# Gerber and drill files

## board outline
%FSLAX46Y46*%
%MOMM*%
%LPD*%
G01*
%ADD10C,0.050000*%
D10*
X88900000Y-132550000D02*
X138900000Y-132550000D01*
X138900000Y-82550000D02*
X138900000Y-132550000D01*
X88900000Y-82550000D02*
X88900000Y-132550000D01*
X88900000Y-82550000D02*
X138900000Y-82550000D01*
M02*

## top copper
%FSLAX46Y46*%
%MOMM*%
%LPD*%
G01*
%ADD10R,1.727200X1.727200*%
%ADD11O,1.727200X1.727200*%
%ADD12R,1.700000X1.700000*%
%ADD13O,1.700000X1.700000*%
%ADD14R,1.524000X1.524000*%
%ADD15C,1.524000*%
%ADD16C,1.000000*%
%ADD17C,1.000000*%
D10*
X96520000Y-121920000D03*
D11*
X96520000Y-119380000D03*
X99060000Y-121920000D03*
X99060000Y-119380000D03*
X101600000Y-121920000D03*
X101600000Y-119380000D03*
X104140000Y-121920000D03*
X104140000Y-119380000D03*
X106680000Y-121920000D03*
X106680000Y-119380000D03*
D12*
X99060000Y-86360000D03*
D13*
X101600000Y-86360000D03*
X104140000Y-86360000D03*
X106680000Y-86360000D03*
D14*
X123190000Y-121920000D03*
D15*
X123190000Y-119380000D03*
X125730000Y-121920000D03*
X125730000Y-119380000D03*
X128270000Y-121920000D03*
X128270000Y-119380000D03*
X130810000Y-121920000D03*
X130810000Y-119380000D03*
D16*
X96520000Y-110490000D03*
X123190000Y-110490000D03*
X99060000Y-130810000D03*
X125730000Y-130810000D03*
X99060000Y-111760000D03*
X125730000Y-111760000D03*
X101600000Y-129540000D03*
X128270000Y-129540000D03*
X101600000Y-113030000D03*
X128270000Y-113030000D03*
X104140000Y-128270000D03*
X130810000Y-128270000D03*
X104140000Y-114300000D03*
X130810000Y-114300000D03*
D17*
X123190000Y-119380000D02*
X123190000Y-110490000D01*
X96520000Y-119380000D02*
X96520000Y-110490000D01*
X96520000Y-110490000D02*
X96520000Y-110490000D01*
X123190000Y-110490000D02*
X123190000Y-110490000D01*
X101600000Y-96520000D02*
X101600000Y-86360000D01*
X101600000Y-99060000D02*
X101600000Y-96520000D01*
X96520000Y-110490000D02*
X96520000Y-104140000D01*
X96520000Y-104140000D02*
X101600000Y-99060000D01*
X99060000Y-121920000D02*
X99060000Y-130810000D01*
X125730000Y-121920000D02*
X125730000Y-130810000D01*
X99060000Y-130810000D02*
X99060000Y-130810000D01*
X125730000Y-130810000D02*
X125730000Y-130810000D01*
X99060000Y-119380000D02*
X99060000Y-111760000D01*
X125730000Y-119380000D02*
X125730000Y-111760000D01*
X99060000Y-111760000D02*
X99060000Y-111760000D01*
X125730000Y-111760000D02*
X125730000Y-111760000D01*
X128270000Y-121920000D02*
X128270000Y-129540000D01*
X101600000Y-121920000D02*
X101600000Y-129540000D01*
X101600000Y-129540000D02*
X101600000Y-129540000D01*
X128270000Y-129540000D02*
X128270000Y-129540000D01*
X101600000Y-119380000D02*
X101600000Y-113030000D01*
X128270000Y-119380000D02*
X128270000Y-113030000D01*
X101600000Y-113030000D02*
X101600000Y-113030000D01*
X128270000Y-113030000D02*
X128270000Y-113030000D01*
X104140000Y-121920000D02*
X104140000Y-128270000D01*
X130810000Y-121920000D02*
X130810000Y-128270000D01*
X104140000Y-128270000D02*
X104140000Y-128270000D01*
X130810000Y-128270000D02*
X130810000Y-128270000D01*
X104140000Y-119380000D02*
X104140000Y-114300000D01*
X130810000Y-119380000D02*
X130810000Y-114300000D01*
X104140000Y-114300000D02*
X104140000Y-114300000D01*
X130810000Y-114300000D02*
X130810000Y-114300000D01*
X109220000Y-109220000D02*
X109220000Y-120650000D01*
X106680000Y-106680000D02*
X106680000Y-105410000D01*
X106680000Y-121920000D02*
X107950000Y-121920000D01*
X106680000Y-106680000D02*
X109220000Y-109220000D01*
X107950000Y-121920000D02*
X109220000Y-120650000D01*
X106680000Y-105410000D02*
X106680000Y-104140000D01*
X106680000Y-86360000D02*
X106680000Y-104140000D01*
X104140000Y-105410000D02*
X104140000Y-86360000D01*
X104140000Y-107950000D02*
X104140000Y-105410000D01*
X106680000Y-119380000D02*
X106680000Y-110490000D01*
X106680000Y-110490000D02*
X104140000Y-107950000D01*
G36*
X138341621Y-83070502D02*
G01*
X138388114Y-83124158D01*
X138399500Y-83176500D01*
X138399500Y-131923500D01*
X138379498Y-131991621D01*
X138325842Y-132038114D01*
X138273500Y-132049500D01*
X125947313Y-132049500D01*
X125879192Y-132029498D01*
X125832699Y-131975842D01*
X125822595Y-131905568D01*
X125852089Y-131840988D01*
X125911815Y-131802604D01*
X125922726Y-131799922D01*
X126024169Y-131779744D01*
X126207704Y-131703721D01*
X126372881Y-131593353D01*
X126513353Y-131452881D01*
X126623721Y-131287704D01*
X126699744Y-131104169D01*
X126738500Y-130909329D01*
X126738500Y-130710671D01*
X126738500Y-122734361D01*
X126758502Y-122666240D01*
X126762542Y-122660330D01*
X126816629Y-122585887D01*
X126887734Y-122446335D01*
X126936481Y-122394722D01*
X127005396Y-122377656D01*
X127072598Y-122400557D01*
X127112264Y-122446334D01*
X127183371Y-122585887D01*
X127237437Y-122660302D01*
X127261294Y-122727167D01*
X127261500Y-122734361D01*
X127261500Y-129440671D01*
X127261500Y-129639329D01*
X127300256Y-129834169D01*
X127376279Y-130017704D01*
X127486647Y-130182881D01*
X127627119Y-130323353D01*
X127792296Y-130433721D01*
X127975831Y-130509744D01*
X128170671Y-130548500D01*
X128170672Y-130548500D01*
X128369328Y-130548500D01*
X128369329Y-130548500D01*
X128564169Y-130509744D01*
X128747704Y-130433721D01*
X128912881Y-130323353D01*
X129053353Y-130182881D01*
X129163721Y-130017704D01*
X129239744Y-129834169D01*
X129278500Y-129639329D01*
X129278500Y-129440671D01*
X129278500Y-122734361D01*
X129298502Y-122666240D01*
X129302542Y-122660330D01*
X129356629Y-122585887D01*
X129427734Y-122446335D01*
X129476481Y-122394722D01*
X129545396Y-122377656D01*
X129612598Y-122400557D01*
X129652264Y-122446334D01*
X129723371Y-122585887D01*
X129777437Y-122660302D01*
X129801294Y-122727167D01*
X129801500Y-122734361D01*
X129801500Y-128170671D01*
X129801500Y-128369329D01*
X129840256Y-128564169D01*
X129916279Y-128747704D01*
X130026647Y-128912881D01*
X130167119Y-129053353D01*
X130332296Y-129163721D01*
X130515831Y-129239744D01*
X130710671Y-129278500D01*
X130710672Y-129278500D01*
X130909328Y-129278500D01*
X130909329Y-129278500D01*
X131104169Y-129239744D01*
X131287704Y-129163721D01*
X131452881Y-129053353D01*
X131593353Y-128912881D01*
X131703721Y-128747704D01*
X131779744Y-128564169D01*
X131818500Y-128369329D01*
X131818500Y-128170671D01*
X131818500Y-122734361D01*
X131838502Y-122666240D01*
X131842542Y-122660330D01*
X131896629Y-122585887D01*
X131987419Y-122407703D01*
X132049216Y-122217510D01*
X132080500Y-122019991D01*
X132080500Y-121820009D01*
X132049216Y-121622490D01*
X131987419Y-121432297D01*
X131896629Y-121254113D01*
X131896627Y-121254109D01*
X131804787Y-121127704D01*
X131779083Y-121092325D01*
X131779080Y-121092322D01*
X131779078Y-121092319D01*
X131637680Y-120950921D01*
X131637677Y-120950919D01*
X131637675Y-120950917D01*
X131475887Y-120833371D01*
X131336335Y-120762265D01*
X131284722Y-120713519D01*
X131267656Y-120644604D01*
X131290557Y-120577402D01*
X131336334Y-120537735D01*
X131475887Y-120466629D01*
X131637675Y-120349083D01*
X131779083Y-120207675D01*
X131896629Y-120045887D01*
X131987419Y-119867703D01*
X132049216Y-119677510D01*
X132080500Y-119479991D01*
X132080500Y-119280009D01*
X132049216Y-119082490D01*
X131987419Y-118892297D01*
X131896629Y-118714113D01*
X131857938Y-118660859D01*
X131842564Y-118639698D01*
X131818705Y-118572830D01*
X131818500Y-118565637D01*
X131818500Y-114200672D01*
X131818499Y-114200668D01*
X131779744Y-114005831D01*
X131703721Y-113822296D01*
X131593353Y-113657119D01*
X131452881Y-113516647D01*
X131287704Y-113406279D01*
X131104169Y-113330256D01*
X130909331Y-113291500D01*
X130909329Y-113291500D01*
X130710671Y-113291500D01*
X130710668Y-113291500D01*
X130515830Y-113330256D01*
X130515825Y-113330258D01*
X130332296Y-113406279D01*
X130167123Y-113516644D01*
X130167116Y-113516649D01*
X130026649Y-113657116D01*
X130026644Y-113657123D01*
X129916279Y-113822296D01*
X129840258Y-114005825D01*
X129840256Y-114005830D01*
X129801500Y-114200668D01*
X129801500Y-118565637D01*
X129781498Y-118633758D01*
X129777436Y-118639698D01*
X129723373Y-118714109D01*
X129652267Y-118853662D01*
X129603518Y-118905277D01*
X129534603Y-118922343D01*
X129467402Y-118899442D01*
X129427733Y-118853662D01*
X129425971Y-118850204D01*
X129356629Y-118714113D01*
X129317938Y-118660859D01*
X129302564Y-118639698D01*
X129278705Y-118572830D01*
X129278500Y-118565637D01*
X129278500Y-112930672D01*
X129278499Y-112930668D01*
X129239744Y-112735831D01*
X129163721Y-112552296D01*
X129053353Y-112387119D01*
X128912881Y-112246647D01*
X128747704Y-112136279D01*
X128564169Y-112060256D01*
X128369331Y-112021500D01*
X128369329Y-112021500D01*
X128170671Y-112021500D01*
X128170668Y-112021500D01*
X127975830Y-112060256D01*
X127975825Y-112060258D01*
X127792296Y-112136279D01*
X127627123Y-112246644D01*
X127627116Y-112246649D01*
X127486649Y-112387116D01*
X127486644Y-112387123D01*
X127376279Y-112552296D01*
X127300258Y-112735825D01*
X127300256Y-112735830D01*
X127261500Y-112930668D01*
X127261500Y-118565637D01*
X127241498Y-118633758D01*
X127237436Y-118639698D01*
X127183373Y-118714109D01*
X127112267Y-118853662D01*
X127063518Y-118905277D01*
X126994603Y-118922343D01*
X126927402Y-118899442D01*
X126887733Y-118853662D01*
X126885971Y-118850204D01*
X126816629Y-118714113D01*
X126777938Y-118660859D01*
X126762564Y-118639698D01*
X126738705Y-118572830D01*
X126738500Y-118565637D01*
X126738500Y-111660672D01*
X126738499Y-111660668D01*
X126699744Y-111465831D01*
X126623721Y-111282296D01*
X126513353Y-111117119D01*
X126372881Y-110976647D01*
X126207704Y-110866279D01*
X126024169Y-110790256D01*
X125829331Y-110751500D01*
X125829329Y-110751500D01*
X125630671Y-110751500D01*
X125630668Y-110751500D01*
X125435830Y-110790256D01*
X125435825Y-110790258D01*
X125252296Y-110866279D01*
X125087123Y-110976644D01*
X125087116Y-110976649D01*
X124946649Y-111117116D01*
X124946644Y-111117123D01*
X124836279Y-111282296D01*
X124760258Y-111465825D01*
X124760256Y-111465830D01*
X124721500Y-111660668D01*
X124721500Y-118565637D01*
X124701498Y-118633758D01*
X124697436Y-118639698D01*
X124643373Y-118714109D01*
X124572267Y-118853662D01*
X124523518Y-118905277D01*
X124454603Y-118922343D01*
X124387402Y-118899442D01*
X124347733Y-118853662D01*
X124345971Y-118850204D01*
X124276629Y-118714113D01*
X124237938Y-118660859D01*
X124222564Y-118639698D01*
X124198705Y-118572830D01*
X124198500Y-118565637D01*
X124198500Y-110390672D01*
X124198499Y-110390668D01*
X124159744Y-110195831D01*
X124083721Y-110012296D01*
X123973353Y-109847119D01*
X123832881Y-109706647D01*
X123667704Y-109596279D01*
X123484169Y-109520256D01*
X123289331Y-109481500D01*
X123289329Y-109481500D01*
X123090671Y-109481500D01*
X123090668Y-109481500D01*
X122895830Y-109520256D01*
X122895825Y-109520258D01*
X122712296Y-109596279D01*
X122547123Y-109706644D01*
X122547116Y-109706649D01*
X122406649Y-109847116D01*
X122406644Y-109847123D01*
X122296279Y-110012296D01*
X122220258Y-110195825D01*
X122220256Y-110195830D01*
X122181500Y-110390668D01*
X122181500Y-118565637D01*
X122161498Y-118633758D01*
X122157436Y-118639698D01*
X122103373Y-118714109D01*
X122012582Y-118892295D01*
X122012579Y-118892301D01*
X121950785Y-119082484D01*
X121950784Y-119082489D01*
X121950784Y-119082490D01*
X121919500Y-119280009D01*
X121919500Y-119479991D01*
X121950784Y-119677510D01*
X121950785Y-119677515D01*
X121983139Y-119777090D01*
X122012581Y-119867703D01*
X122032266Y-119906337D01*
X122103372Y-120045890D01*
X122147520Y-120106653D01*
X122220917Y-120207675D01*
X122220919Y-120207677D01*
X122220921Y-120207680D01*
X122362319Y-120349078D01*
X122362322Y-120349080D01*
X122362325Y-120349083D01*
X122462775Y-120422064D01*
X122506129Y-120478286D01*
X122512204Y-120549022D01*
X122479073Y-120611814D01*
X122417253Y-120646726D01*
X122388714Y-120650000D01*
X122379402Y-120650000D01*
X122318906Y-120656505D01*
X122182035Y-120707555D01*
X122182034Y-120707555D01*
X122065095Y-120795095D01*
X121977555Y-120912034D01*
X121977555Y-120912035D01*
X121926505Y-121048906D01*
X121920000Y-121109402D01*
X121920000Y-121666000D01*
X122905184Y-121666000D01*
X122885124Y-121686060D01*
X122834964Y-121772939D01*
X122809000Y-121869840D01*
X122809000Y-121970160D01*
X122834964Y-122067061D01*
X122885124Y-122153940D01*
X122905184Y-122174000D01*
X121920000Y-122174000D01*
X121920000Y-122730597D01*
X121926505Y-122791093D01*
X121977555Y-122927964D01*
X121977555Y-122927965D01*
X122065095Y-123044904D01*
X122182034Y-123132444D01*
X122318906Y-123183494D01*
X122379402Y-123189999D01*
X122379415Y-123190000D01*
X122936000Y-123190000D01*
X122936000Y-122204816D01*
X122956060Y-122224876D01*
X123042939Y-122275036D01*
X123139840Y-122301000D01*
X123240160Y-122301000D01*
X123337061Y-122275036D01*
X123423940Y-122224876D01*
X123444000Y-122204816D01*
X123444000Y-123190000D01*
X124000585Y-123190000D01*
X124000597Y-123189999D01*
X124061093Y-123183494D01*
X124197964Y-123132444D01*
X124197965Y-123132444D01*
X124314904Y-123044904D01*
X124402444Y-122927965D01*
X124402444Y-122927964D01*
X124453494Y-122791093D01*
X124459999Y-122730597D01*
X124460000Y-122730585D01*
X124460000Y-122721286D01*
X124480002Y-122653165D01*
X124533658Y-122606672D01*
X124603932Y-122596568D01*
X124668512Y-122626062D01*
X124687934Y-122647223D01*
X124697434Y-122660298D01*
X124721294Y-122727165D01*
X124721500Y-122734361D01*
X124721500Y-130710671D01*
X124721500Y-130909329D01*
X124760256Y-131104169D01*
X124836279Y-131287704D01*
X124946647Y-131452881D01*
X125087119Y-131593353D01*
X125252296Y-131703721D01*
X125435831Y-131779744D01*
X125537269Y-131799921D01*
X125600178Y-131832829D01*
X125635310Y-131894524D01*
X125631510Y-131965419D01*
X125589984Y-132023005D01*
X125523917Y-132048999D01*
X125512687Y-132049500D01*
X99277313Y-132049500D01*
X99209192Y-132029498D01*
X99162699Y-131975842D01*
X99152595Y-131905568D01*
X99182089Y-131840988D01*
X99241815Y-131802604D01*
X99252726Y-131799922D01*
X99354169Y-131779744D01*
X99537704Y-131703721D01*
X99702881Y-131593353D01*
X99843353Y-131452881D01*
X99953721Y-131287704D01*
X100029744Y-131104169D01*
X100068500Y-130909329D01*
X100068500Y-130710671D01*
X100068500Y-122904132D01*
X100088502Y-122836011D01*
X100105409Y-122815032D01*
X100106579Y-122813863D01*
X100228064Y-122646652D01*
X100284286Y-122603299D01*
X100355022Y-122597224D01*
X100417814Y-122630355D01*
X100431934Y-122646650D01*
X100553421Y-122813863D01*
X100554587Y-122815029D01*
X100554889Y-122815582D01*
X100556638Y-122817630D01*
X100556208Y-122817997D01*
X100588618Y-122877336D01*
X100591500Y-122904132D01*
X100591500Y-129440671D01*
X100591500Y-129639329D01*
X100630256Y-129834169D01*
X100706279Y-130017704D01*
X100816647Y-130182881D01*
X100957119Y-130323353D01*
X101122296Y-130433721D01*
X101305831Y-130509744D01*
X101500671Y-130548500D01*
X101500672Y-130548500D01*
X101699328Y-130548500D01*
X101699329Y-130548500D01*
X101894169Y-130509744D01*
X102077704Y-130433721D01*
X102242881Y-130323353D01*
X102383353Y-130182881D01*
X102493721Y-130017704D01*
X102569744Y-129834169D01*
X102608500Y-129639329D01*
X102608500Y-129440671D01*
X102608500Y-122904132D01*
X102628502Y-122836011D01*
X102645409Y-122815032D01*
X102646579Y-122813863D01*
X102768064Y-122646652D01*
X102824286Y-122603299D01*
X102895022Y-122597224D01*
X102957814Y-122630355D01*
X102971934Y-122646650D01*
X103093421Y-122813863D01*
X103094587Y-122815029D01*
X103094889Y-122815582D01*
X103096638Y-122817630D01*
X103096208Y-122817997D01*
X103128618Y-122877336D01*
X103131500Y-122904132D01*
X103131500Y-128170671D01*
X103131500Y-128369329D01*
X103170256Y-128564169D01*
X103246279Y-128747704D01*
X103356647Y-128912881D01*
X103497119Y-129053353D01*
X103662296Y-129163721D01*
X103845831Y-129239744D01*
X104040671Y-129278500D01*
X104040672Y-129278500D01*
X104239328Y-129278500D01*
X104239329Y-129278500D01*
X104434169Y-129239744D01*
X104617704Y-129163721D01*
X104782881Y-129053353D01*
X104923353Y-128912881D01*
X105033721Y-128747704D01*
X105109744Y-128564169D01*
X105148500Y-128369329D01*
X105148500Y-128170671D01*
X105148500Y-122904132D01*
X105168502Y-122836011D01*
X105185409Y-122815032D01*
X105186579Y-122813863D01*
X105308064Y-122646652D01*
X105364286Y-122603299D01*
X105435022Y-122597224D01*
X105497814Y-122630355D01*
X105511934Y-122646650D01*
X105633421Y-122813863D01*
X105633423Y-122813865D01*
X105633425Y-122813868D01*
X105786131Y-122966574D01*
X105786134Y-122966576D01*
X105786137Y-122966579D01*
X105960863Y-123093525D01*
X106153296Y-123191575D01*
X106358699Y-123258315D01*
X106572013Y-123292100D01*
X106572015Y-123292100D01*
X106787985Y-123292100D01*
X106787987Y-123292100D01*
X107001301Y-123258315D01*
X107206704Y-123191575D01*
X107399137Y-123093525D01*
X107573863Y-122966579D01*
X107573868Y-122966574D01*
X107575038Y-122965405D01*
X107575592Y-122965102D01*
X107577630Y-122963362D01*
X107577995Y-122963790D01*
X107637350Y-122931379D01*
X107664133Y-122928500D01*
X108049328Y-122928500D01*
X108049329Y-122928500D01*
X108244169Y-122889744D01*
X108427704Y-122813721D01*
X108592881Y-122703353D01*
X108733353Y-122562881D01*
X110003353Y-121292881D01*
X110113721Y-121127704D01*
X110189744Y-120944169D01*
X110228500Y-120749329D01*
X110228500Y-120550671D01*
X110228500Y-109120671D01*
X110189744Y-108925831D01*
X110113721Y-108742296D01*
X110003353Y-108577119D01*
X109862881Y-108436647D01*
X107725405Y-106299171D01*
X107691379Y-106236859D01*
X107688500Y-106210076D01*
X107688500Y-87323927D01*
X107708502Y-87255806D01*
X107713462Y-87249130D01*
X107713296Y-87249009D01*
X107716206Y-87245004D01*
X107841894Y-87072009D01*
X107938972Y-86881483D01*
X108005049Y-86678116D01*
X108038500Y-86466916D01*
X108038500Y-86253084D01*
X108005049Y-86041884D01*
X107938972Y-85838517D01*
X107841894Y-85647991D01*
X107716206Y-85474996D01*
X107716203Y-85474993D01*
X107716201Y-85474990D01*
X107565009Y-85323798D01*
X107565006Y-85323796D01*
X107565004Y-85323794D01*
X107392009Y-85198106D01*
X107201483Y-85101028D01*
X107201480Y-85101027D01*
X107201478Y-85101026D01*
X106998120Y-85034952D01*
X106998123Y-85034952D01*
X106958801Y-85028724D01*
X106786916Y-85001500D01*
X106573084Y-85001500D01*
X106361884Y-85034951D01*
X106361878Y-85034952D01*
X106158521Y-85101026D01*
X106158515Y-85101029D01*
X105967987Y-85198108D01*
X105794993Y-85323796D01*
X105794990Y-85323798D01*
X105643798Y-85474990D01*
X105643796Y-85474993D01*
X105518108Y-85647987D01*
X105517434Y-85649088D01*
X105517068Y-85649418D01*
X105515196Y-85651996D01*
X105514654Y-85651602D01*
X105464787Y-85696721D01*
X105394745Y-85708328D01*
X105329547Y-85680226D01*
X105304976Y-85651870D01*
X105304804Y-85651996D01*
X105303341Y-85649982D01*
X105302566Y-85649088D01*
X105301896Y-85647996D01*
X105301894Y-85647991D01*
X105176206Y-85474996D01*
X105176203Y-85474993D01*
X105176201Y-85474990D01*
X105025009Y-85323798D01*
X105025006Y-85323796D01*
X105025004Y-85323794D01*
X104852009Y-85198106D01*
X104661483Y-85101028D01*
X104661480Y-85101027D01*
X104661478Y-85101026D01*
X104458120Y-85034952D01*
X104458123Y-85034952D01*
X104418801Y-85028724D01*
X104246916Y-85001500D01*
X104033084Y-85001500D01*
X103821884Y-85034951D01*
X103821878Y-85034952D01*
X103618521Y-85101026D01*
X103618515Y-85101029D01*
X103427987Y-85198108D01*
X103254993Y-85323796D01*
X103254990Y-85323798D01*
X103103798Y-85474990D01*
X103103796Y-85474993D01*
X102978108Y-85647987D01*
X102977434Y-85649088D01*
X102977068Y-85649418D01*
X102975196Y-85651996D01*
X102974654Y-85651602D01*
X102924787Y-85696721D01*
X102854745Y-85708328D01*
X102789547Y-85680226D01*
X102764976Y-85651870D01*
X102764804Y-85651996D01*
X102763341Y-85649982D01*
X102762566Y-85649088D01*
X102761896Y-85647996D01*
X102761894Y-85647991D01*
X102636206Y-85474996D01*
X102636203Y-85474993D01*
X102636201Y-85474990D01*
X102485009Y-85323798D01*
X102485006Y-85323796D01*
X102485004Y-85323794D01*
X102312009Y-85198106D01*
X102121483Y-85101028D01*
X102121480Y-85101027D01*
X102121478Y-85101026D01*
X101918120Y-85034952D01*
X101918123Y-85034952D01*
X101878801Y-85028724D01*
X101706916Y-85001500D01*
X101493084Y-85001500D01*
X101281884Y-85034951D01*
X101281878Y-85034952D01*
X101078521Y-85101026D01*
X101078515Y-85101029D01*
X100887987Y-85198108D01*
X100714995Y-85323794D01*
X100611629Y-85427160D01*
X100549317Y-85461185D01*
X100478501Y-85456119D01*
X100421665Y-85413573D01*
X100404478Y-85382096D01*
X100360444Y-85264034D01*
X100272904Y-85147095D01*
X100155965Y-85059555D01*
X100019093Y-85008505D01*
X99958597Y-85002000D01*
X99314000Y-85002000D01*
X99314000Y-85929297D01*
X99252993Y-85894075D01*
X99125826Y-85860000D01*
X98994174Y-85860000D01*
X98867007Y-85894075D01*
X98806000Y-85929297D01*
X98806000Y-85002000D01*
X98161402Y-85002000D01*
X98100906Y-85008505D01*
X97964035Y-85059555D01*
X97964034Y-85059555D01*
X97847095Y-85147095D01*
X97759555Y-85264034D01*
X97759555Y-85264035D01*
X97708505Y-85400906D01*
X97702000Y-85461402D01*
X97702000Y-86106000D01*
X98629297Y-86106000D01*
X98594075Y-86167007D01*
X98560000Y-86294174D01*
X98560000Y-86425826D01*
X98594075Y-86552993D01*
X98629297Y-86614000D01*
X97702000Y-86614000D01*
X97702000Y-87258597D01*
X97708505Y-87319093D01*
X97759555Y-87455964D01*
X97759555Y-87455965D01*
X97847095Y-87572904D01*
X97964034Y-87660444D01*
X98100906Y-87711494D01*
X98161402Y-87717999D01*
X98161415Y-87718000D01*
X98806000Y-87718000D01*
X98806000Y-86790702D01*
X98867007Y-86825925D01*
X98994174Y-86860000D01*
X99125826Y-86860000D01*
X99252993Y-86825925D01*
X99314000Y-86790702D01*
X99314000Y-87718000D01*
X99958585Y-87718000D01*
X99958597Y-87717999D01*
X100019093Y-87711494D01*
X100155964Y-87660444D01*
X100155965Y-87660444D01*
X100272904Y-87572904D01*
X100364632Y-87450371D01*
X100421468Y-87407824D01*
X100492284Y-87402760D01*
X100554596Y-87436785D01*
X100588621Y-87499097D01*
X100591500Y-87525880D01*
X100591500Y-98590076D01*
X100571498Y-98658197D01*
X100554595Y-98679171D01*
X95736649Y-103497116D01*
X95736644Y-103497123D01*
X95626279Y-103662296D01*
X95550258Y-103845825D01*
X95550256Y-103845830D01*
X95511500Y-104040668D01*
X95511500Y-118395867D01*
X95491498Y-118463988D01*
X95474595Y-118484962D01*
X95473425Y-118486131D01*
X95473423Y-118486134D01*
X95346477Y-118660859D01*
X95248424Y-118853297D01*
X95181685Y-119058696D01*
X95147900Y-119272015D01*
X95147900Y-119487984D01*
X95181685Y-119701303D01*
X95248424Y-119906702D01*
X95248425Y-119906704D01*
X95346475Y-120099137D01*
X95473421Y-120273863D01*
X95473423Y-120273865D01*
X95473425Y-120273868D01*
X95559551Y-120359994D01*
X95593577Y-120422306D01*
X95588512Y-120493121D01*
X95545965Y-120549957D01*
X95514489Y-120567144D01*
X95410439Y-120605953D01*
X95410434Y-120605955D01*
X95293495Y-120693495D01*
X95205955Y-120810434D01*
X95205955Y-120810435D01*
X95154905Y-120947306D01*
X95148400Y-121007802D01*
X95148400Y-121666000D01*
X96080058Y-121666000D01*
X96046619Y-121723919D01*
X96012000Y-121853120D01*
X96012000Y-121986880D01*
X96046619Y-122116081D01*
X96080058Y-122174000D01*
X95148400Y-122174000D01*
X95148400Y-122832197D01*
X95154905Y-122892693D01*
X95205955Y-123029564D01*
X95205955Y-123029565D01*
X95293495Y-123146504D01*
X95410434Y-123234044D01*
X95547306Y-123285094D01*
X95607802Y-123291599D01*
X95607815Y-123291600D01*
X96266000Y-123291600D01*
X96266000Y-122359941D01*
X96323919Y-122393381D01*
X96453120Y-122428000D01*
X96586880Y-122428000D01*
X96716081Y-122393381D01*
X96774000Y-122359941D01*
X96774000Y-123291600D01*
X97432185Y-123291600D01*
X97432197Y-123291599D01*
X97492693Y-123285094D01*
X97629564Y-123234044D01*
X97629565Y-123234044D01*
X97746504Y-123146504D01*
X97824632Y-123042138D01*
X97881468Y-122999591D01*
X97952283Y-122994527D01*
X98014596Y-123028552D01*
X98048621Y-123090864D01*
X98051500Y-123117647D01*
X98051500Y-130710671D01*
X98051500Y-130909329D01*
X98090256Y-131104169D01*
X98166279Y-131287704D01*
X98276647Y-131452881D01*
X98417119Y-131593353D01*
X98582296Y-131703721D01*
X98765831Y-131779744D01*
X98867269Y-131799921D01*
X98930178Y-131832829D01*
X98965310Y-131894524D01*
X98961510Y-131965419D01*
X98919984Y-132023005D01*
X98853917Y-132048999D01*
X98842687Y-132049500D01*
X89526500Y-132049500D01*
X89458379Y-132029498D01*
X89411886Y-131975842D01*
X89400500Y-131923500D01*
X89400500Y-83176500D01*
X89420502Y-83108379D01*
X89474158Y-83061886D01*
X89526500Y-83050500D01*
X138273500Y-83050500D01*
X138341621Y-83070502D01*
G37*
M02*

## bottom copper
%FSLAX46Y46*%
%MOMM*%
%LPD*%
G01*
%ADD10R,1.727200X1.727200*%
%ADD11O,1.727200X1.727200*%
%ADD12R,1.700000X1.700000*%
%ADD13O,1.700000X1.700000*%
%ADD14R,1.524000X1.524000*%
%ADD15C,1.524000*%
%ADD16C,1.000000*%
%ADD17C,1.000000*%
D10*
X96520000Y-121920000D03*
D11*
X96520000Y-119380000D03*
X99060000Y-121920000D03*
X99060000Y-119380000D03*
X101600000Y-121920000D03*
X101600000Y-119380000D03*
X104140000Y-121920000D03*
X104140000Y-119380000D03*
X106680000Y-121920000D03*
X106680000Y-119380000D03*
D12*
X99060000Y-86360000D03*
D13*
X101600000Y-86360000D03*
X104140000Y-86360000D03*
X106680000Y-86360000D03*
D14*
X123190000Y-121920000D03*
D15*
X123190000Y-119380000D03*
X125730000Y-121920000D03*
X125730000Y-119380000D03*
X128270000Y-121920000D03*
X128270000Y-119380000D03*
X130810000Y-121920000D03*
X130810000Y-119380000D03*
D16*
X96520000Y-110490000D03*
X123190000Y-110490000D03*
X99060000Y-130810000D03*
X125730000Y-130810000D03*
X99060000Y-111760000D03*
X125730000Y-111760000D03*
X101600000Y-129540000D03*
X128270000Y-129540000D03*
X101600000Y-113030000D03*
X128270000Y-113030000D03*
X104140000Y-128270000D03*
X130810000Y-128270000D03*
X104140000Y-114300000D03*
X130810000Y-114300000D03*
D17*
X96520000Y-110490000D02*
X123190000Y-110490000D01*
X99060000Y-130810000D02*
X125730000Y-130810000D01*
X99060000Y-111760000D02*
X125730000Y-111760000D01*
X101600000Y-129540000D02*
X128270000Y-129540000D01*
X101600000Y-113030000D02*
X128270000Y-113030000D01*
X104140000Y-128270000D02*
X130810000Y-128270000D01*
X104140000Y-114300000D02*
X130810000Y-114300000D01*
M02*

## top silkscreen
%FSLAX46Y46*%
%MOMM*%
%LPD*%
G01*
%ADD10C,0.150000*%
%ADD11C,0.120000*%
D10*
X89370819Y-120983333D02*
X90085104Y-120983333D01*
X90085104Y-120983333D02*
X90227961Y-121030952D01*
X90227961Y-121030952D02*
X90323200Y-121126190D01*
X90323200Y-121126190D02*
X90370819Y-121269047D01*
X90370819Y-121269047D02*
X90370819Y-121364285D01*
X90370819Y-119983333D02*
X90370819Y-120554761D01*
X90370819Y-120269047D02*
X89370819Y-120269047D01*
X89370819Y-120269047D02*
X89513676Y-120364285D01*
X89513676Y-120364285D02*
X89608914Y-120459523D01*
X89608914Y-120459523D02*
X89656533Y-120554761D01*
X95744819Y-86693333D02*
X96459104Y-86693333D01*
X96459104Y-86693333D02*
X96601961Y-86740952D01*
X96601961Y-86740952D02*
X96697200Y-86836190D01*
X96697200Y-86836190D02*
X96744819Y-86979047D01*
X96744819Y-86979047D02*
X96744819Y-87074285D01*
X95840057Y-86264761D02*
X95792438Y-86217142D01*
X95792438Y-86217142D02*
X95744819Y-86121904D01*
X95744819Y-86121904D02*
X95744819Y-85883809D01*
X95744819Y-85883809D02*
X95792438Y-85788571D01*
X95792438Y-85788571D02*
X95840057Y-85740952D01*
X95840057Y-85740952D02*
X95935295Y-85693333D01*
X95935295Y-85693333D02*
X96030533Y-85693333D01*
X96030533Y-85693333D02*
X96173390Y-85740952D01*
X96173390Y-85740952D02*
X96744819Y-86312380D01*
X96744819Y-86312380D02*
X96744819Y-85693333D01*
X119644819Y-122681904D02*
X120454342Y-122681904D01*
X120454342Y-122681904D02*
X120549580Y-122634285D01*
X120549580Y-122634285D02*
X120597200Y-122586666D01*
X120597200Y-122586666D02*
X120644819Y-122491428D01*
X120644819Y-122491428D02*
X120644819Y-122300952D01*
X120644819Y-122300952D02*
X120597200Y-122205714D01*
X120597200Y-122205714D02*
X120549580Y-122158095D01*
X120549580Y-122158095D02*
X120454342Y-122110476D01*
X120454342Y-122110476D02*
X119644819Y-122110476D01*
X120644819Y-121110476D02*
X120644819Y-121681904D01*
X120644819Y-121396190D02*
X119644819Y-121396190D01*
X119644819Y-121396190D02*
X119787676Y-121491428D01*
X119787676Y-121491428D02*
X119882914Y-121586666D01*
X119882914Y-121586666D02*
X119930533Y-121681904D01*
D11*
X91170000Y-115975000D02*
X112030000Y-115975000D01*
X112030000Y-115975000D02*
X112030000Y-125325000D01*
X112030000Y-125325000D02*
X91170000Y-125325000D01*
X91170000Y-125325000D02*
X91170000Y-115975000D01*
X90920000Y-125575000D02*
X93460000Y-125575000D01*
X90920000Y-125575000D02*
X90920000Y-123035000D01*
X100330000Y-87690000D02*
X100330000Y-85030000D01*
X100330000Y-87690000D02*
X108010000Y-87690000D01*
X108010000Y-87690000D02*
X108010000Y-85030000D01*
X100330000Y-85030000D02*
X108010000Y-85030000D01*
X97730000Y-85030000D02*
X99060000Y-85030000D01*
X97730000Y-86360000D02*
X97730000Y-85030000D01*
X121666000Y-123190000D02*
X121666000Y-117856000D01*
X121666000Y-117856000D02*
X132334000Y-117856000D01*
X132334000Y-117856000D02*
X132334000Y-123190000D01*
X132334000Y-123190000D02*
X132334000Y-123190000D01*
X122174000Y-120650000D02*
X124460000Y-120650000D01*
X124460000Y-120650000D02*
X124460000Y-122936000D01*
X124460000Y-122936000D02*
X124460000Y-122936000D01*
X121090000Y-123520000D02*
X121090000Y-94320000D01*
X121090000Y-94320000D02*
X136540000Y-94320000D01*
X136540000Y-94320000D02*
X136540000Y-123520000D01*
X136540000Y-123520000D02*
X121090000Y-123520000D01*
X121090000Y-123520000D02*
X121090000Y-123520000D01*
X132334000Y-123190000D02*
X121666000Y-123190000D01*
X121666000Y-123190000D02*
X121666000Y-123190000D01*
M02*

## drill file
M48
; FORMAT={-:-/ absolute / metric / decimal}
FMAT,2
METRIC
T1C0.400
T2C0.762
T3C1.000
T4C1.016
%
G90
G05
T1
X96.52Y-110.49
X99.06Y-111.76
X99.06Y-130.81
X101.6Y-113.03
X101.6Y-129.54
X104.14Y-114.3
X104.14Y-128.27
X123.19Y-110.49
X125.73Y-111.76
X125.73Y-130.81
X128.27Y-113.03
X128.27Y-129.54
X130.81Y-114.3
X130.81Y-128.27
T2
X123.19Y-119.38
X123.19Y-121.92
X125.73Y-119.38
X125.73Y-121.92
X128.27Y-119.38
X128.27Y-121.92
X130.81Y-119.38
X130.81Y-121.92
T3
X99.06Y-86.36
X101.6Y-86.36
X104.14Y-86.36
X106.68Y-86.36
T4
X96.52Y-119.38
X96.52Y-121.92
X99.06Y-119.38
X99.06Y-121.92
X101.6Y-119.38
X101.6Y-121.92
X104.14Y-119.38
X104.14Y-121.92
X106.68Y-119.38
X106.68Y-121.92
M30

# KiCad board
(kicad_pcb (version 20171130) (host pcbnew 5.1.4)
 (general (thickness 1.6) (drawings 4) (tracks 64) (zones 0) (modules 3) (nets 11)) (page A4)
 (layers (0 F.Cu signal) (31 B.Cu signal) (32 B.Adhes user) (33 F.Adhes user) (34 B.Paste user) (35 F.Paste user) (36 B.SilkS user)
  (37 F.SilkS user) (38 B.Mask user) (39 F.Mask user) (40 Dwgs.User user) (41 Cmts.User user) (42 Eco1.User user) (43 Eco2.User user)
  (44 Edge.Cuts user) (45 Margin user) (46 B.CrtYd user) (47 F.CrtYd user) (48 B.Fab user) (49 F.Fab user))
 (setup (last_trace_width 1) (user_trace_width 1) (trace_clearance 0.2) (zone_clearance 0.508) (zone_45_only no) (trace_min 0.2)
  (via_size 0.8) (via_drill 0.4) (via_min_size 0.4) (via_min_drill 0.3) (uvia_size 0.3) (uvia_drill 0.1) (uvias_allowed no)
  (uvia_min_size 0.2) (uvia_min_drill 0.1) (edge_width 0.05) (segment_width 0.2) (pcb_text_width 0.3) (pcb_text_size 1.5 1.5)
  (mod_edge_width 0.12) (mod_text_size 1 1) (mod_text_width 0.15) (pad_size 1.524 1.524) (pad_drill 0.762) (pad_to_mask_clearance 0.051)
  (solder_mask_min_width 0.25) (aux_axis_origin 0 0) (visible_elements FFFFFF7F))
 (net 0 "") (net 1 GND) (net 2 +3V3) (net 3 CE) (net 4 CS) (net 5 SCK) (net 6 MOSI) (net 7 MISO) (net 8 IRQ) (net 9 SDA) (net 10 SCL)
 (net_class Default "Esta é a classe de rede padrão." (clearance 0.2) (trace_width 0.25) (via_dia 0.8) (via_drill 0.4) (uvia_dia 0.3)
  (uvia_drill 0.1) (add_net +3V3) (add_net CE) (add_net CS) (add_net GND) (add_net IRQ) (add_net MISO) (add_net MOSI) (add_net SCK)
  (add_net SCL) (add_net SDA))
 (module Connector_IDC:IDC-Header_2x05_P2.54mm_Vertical (layer F.Cu) (at 96.52 121.92 90)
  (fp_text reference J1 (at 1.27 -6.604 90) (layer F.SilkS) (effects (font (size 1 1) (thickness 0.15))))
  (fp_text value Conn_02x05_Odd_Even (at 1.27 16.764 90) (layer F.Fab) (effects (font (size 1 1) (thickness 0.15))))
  (fp_line (start 5.945 -5.35) (end 5.945 15.51) (layer F.SilkS) (width 0.12))
  (fp_line (start 5.945 15.51) (end -3.405 15.51) (layer F.SilkS) (width 0.12))
  (fp_line (start -3.405 15.51) (end -3.405 -5.35) (layer F.SilkS) (width 0.12))
  (fp_line (start -3.405 -5.35) (end 5.945 -5.35) (layer F.SilkS) (width 0.12))
  (fp_line (start -3.655 -5.6) (end -3.655 -3.06) (layer F.SilkS) (width 0.12))
  (fp_line (start -3.655 -5.6) (end -1.115 -5.6) (layer F.SilkS) (width 0.12))
  (pad 1 thru_hole rect (at 0 0 90) (size 1.7272 1.7272) (drill 1.016) (layers *.Cu *.Mask) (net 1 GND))
  (pad 2 thru_hole oval (at 2.54 0 90) (size 1.7272 1.7272) (drill 1.016) (layers *.Cu *.Mask) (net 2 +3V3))
  (pad 3 thru_hole oval (at 0 2.54 90) (size 1.7272 1.7272) (drill 1.016) (layers *.Cu *.Mask) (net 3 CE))
  (pad 4 thru_hole oval (at 2.54 2.54 90) (size 1.7272 1.7272) (drill 1.016) (layers *.Cu *.Mask) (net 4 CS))
  (pad 5 thru_hole oval (at 0 5.08 90) (size 1.7272 1.7272) (drill 1.016) (layers *.Cu *.Mask) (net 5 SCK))
  (pad 6 thru_hole oval (at 2.54 5.08 90) (size 1.7272 1.7272) (drill 1.016) (layers *.Cu *.Mask) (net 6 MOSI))
  (pad 7 thru_hole oval (at 0 7.62 90) (size 1.7272 1.7272) (drill 1.016) (layers *.Cu *.Mask) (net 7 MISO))
  (pad 8 thru_hole oval (at 2.54 7.62 90) (size 1.7272 1.7272) (drill 1.016) (layers *.Cu *.Mask) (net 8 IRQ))
  (pad 9 thru_hole oval (at 0 10.16 90) (size 1.7272 1.7272) (drill 1.016) (layers *.Cu *.Mask) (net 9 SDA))
  (pad 10 thru_hole oval (at 2.54 10.16 90) (size 1.7272 1.7272) (drill 1.016) (layers *.Cu *.Mask) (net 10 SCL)))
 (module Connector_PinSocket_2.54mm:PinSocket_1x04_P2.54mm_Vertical (layer F.Cu) (at 99.06 86.36 90)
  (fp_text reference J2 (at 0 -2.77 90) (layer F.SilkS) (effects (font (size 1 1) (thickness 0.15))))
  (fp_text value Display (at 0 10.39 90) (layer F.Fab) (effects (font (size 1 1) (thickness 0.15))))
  (fp_line (start -1.33 1.27) (end 1.33 1.27) (layer F.SilkS) (width 0.12))
  (fp_line (start -1.33 1.27) (end -1.33 8.95) (layer F.SilkS) (width 0.12))
  (fp_line (start -1.33 8.95) (end 1.33 8.95) (layer F.SilkS) (width 0.12))
  (fp_line (start 1.33 1.27) (end 1.33 8.95) (layer F.SilkS) (width 0.12))
  (fp_line (start 1.33 -1.33) (end 1.33 0) (layer F.SilkS) (width 0.12))
  (fp_line (start 0 -1.33) (end 1.33 -1.33) (layer F.SilkS) (width 0.12))
  (pad 1 thru_hole rect (at 0 0 90) (size 1.7 1.7) (drill 1) (layers *.Cu *.Mask) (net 1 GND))
  (pad 2 thru_hole oval (at 0 2.54 90) (size 1.7 1.7) (drill 1) (layers *.Cu *.Mask) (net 2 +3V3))
  (pad 3 thru_hole oval (at 0 5.08 90) (size 1.7 1.7) (drill 1) (layers *.Cu *.Mask) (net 10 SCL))
  (pad 4 thru_hole oval (at 0 7.62 90) (size 1.7 1.7) (drill 1) (layers *.Cu *.Mask) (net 9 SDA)))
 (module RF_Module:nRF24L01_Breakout (layer F.Cu) (at 123.19 121.92 90)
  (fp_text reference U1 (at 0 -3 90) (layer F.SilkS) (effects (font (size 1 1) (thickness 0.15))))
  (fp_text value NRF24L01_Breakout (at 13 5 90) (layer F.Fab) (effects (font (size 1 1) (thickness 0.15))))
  (fp_line (start -1.27 -1.524) (end 4.064 -1.524) (layer F.SilkS) (width 0.12))
  (fp_line (start 4.064 -1.524) (end 4.064 9.144) (layer F.SilkS) (width 0.12))
  (fp_line (start 4.064 9.144) (end -1.27 9.144) (layer F.SilkS) (width 0.12))
  (fp_line (start -1.27 9.144) (end -1.27 9.144) (layer F.SilkS) (width 0.12))
  (fp_line (start 1.27 -1.016) (end 1.27 1.27) (layer F.SilkS) (width 0.12))
  (fp_line (start 1.27 1.27) (end -1.016 1.27) (layer F.SilkS) (width 0.12))
  (fp_line (start -1.016 1.27) (end -1.016 1.27) (layer F.SilkS) (width 0.12))
  (fp_line (start -1.6 -2.1) (end 27.6 -2.1) (layer F.SilkS) (width 0.12))
  (fp_line (start 27.6 -2.1) (end 27.6 13.35) (layer F.SilkS) (width 0.12))
  (fp_line (start 27.6 13.35) (end -1.6 13.35) (layer F.SilkS) (width 0.12))
  (fp_line (start -1.6 13.35) (end -1.6 -2.1) (layer F.SilkS) (width 0.12))
  (fp_line (start -1.6 -2.1) (end -1.6 -2.1) (layer F.SilkS) (width 0.12))
  (fp_line (start -1.27 9.144) (end -1.27 -1.524) (layer F.SilkS) (width 0.12))
  (fp_line (start -1.27 -1.524) (end -1.27 -1.524) (layer F.SilkS) (width 0.12))
  (pad 1 thru_hole rect (at 0 0 90) (size 1.524 1.524) (drill 0.762) (layers *.Cu *.Mask) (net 1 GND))
  (pad 2 thru_hole circle (at 2.54 0 90) (size 1.524 1.524) (drill 0.762) (layers *.Cu *.Mask) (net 2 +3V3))
  (pad 3 thru_hole circle (at 0 2.54 90) (size 1.524 1.524) (drill 0.762) (layers *.Cu *.Mask) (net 3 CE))
  (pad 4 thru_hole circle (at 2.54 2.54 90) (size 1.524 1.524) (drill 0.762) (layers *.Cu *.Mask) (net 4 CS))
  (pad 5 thru_hole circle (at 0 5.08 90) (size 1.524 1.524) (drill 0.762) (layers *.Cu *.Mask) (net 5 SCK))
  (pad 6 thru_hole circle (at 2.54 5.08 90) (size 1.524 1.524) (drill 0.762) (layers *.Cu *.Mask) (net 6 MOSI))
  (pad 7 thru_hole circle (at 0 7.62 90) (size 1.524 1.524) (drill 0.762) (layers *.Cu *.Mask) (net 7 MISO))
  (pad 8 thru_hole circle (at 2.54 7.62 90) (size 1.524 1.524) (drill 0.762) (layers *.Cu *.Mask) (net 8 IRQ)))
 (gr_line (start 88.9 132.55) (end 138.9 132.55) (layer Edge.Cuts) (width 0.05))
 (gr_line (start 138.9 82.55) (end 138.9 132.55) (layer Edge.Cuts) (width 0.05))
 (gr_line (start 88.9 82.55) (end 88.9 132.55) (layer Edge.Cuts) (width 0.05))
 (gr_line (start 88.9 82.55) (end 138.9 82.55) (layer Edge.Cuts) (width 0.05))
 (segment (start 123.19 119.38) (end 123.19 110.49) (width 1) (layer F.Cu) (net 2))
 (segment (start 96.52 119.38) (end 96.52 110.49) (width 1) (layer F.Cu) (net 2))
 (segment (start 96.52 110.49) (end 96.52 110.49) (width 1) (layer F.Cu) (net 2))
 (via (at 96.52 110.49) (size 1) (drill 0.4) (layers F.Cu B.Cu) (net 2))
 (segment (start 123.19 110.49) (end 123.19 110.49) (width 1) (layer F.Cu) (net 2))
 (via (at 123.19 110.49) (size 1) (drill 0.4) (layers F.Cu B.Cu) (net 2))
 (segment (start 96.52 110.49) (end 123.19 110.49) (width 1) (layer B.Cu) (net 2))
 (segment (start 101.6 96.52) (end 101.6 86.36) (width 1) (layer F.Cu) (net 2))
 (segment (start 101.6 99.06) (end 101.6 96.52) (width 1) (layer F.Cu) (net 2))
 (segment (start 96.52 110.49) (end 96.52 104.14) (width 1) (layer F.Cu) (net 2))
 (segment (start 96.52 104.14) (end 101.6 99.06) (width 1) (layer F.Cu) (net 2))
 (segment (start 99.06 121.92) (end 99.06 130.81) (width 1) (layer F.Cu) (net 3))
 (segment (start 125.73 121.92) (end 125.73 130.81) (width 1) (layer F.Cu) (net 3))
 (segment (start 99.06 130.81) (end 99.06 130.81) (width 1) (layer F.Cu) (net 3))
 (via (at 99.06 130.81) (size 1) (drill 0.4) (layers F.Cu B.Cu) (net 3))
 (segment (start 125.73 130.81) (end 125.73 130.81) (width 1) (layer F.Cu) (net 3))
 (via (at 125.73 130.81) (size 1) (drill 0.4) (layers F.Cu B.Cu) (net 3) (status 1000000))
 (segment (start 99.06 130.81) (end 125.73 130.81) (width 1) (layer B.Cu) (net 3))
 (segment (start 99.06 119.38) (end 99.06 111.76) (width 1) (layer F.Cu) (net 4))
 (segment (start 125.73 119.38) (end 125.73 111.76) (width 1) (layer F.Cu) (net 4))
 (segment (start 99.06 111.76) (end 99.06 111.76) (width 1) (layer F.Cu) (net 4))
 (via (at 99.06 111.76) (size 1) (drill 0.4) (layers F.Cu B.Cu) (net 4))
 (segment (start 125.73 111.76) (end 125.73 111.76) (width 1) (layer F.Cu) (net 4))
 (via (at 125.73 111.76) (size 1) (drill 0.4) (layers F.Cu B.Cu) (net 4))
 (segment (start 99.06 111.76) (end 125.73 111.76) (width 1) (layer B.Cu) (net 4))
 (segment (start 128.27 121.92) (end 128.27 129.54) (width 1) (layer F.Cu) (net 5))
 (segment (start 101.6 121.92) (end 101.6 129.54) (width 1) (layer F.Cu) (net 5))
 (segment (start 101.6 129.54) (end 101.6 129.54) (width 1) (layer F.Cu) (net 5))
 (via (at 101.6 129.54) (size 1) (drill 0.4) (layers F.Cu B.Cu) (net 5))
 (segment (start 128.27 129.54) (end 128.27 129.54) (width 1) (layer F.Cu) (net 5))
 (via (at 128.27 129.54) (size 1) (drill 0.4) (layers F.Cu B.Cu) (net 5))
 (segment (start 101.6 129.54) (end 128.27 129.54) (width 1) (layer B.Cu) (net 5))
 (segment (start 101.6 119.38) (end 101.6 113.03) (width 1) (layer F.Cu) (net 6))
 (segment (start 128.27 119.38) (end 128.27 113.03) (width 1) (layer F.Cu) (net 6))
 (segment (start 101.6 113.03) (end 101.6 113.03) (width 1) (layer F.Cu) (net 6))
 (via (at 101.6 113.03) (size 1) (drill 0.4) (layers F.Cu B.Cu) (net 6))
 (segment (start 128.27 113.03) (end 128.27 113.03) (width 1) (layer F.Cu) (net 6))
 (via (at 128.27 113.03) (size 1) (drill 0.4) (layers F.Cu B.Cu) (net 6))
 (segment (start 101.6 113.03) (end 128.27 113.03) (width 1) (layer B.Cu) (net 6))
 (segment (start 104.14 121.92) (end 104.14 128.27) (width 1) (layer F.Cu) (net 7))
 (segment (start 130.81 121.92) (end 130.81 128.27) (width 1) (layer F.Cu) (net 7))
 (segment (start 104.14 128.27) (end 104.14 128.27) (width 1) (layer F.Cu) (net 7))
 (via (at 104.14 128.27) (size 1) (drill 0.4) (layers F.Cu B.Cu) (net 7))
 (segment (start 130.81 128.27) (end 130.81 128.27) (width 1) (layer F.Cu) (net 7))
 (via (at 130.81 128.27) (size 1) (drill 0.4) (layers F.Cu B.Cu) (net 7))
 (segment (start 104.14 128.27) (end 130.81 128.27) (width 1) (layer B.Cu) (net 7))
 (segment (start 104.14 119.38) (end 104.14 114.3) (width 1) (layer F.Cu) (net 8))
 (segment (start 130.81 119.38) (end 130.81 114.3) (width 1) (layer F.Cu) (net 8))
 (segment (start 104.14 114.3) (end 104.14 114.3) (width 1) (layer F.Cu) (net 8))
 (via (at 104.14 114.3) (size 1) (drill 0.4) (layers F.Cu B.Cu) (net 8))
 (segment (start 130.81 114.3) (end 130.81 114.3) (width 1) (layer F.Cu) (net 8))
 (via (at 130.81 114.3) (size 1) (drill 0.4) (layers F.Cu B.Cu) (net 8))
 (segment (start 104.14 114.3) (end 130.81 114.3) (width 1) (layer B.Cu) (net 8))
 (segment (start 109.22 109.22) (end 109.22 120.65) (width 1) (layer F.Cu) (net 9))
 (segment (start 106.68 106.68) (end 106.68 105.41) (width 1) (layer F.Cu) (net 9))
 (segment (start 106.68 121.92) (end 107.95 121.92) (width 1) (layer F.Cu) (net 9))
 (segment (start 106.68 106.68) (end 109.22 109.22) (width 1) (layer F.Cu) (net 9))
 (segment (start 107.95 121.92) (end 109.22 120.65) (width 1) (layer F.Cu) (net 9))
 (segment (start 106.68 105.41) (end 106.68 104.14) (width 1) (layer F.Cu) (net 9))
 (segment (start 106.68 86.36) (end 106.68 104.14) (width 1) (layer F.Cu) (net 9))
 (segment (start 104.14 105.41) (end 104.14 86.36) (width 1) (layer F.Cu) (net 10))
 (segment (start 104.14 107.95) (end 104.14 105.41) (width 1) (layer F.Cu) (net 10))
 (segment (start 106.68 119.38) (end 106.68 110.49) (width 1) (layer F.Cu) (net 10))
 (segment (start 106.68 110.49) (end 104.14 107.95) (width 1) (layer F.Cu) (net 10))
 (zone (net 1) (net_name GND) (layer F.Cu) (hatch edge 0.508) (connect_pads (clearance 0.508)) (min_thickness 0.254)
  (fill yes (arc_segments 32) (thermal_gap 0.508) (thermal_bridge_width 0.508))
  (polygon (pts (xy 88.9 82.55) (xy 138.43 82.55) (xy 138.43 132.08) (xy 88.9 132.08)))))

